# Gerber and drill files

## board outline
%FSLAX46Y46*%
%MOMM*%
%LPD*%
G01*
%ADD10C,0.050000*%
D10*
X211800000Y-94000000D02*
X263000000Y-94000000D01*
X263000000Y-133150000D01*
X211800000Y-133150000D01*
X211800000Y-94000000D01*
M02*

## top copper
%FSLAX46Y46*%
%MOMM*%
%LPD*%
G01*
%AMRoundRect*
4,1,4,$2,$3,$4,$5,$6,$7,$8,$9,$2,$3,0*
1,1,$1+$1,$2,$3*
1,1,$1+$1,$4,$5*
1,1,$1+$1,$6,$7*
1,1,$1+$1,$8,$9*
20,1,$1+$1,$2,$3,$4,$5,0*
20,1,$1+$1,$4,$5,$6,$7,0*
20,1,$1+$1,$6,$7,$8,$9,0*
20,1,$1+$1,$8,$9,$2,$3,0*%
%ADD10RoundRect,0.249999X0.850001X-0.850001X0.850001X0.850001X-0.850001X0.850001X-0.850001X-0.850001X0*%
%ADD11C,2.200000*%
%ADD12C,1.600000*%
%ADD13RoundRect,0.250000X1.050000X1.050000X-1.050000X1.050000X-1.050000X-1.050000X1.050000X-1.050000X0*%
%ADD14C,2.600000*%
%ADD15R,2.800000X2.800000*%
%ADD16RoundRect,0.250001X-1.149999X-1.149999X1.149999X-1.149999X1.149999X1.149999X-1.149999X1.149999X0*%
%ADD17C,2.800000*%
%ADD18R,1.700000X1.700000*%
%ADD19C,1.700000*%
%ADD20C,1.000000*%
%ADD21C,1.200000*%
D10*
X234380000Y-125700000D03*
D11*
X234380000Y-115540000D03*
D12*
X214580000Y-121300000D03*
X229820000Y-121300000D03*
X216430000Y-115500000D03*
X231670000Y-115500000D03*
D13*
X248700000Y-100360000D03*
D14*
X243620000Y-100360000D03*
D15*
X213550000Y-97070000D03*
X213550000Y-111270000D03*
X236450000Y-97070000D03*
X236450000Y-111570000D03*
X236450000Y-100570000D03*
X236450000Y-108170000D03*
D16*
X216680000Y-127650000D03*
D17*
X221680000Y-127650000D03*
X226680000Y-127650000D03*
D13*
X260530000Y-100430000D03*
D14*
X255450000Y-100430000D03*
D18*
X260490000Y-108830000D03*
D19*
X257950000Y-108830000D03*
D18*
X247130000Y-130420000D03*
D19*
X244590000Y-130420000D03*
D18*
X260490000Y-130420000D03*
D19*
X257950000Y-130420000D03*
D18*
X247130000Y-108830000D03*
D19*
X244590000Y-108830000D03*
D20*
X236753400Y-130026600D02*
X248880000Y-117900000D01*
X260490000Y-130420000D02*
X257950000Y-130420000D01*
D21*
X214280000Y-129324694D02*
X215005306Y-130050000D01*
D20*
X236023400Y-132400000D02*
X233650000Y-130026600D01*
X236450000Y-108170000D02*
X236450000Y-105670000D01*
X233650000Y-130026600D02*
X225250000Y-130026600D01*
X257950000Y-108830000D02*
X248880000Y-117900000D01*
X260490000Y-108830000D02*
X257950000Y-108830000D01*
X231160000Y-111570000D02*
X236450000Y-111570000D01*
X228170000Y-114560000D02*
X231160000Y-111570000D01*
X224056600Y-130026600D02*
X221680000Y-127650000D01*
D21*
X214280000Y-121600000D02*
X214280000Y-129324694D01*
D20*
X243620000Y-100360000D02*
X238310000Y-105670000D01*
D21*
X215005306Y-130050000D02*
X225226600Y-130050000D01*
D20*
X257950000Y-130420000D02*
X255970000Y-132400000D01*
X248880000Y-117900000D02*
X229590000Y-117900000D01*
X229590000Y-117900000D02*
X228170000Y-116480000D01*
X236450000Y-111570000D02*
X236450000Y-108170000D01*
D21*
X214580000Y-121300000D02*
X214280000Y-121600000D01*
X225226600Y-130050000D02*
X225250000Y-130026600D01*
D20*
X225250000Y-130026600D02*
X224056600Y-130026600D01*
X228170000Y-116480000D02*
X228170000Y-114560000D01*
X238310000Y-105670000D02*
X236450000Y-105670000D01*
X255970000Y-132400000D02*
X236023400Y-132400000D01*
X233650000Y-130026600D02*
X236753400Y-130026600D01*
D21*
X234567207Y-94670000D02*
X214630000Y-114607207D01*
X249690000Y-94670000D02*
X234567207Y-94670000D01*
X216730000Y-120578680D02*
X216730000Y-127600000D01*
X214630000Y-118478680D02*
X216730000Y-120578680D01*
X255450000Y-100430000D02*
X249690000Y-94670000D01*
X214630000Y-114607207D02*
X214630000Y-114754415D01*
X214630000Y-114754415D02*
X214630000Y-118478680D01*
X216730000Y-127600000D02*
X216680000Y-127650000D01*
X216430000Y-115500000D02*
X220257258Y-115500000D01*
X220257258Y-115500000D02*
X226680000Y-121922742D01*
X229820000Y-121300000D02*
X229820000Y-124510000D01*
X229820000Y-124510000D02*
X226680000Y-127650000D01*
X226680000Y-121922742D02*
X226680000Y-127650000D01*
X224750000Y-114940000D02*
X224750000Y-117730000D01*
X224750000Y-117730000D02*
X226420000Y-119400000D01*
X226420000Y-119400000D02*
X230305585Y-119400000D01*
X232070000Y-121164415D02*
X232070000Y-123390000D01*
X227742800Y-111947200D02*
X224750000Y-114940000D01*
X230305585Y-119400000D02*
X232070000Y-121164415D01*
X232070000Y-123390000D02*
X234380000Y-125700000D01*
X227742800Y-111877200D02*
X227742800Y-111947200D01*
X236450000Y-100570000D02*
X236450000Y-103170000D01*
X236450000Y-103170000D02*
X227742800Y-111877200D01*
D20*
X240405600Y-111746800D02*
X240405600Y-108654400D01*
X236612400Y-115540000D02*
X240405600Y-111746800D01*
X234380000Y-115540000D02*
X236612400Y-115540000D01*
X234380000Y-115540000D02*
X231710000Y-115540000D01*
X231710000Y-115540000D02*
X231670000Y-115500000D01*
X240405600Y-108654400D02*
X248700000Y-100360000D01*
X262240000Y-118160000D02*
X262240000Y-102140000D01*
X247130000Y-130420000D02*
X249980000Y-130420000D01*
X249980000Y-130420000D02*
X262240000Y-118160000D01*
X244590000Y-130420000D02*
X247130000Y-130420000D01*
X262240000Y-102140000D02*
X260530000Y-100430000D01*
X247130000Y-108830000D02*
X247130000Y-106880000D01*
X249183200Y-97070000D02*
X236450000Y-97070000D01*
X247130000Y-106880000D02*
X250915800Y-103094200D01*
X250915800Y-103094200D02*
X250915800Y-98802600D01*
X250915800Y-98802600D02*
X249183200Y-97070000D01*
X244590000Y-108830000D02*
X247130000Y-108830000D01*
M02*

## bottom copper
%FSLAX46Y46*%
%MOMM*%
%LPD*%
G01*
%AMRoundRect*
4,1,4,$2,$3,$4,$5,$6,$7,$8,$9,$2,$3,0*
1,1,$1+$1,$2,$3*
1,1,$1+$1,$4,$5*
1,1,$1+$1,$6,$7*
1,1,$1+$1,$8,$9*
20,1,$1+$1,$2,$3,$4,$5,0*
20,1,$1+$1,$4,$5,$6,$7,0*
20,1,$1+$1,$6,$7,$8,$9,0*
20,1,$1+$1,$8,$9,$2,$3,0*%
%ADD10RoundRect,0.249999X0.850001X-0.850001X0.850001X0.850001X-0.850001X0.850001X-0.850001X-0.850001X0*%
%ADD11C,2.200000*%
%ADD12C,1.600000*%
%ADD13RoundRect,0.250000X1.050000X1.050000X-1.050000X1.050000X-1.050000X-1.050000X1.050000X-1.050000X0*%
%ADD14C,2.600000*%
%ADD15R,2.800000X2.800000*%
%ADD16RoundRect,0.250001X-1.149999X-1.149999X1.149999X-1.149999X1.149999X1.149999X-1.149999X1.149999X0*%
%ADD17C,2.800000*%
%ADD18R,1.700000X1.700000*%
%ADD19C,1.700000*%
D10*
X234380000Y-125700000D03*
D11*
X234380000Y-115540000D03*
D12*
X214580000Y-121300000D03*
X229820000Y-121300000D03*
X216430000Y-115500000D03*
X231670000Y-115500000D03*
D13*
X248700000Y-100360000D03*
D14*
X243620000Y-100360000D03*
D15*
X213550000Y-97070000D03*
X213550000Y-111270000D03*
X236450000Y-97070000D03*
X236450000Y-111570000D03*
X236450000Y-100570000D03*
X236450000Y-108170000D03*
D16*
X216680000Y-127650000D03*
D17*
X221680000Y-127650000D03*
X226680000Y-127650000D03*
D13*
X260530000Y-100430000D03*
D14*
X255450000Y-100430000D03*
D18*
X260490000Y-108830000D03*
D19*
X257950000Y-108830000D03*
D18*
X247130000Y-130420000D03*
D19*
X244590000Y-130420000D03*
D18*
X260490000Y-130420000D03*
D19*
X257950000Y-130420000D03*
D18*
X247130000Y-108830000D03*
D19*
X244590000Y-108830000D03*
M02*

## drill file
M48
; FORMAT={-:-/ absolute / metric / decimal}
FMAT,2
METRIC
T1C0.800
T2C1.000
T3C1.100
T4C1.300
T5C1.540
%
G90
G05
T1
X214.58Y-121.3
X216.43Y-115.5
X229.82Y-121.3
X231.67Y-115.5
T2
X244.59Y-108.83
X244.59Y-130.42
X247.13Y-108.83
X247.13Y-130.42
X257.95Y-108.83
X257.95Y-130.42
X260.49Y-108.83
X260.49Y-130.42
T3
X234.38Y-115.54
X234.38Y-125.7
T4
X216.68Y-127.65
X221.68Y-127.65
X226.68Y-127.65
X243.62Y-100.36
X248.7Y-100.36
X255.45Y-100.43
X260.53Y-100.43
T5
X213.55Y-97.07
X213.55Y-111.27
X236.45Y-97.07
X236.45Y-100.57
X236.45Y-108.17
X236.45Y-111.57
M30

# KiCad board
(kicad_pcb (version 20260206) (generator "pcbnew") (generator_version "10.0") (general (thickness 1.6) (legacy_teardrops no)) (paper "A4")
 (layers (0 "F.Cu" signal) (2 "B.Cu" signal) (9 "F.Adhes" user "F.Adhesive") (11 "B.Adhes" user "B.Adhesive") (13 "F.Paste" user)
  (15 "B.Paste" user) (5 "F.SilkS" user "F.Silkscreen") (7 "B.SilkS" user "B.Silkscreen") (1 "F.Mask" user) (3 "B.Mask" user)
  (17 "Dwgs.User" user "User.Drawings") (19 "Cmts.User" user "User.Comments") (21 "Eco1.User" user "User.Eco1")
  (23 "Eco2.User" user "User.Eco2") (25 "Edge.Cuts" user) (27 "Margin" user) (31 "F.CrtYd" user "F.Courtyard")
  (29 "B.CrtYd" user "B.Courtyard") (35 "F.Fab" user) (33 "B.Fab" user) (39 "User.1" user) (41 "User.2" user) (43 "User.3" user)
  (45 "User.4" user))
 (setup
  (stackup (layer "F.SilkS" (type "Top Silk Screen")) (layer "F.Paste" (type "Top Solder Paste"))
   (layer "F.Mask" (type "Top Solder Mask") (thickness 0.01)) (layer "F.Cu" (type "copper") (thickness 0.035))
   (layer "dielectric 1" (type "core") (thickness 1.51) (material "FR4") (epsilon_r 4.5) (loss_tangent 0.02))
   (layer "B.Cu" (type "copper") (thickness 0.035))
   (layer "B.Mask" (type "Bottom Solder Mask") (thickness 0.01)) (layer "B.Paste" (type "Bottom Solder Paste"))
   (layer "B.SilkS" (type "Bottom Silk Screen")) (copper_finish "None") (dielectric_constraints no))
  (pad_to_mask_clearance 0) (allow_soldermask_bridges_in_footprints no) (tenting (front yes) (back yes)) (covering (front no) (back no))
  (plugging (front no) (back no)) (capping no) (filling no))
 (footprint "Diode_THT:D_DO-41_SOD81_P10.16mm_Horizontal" (layer "F.Cu") (at 234.38 125.7 90)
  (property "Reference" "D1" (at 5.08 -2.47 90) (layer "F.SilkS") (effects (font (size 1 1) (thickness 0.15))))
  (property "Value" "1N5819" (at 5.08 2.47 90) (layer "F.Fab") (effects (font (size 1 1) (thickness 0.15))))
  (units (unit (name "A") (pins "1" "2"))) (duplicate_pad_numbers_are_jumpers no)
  (pad "1" thru_hole roundrect (at 0 0 90) (size 2.2 2.2) (drill 1.1) (layers "*.Cu" "*.Mask") (remove_unused_layers no)
   (roundrect_rratio 0.113636) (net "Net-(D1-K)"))
  (pad "2" thru_hole circle (at 10.16 0 90) (size 2.2 2.2) (drill 1.1) (layers "*.Cu" "*.Mask") (remove_unused_layers no) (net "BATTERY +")))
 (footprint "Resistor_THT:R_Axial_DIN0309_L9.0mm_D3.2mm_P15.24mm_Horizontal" (layer "F.Cu") (at 214.58 121.3)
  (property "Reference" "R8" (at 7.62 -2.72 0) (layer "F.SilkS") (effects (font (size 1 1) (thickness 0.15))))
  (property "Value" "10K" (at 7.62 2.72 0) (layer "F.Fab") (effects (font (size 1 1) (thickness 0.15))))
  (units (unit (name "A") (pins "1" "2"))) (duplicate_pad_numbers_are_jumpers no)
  (pad "1" thru_hole circle (at 0 0) (size 1.6 1.6) (drill 0.8) (layers "*.Cu" "*.Mask") (remove_unused_layers no) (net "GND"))
  (pad "2" thru_hole circle (at 15.24 0) (size 1.6 1.6) (drill 0.8) (layers "*.Cu" "*.Mask") (remove_unused_layers no) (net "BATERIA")))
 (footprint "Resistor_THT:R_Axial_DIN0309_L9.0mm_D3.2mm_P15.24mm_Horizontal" (layer "F.Cu") (at 216.43 115.5)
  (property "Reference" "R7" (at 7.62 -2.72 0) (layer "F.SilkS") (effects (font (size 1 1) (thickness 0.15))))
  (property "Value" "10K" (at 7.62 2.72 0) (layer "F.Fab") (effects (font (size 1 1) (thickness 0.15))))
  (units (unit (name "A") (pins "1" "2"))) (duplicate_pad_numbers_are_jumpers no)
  (pad "1" thru_hole circle (at 0 0) (size 1.6 1.6) (drill 0.8) (layers "*.Cu" "*.Mask") (remove_unused_layers no) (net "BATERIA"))
  (pad "2" thru_hole circle (at 15.24 0) (size 1.6 1.6) (drill 0.8) (layers "*.Cu" "*.Mask") (remove_unused_layers no) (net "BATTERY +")))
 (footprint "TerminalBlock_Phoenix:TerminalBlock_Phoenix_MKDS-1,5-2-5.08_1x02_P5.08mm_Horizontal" (layer "F.Cu") (at 248.7 100.36 180)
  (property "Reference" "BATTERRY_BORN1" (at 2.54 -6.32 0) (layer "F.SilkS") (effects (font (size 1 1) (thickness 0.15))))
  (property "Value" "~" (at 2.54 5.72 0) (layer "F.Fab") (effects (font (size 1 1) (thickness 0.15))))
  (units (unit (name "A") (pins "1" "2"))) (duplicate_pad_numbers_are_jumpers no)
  (pad "1" thru_hole roundrect (at 0 0 180) (size 2.6 2.6) (drill 1.3) (layers "*.Cu" "*.Mask") (remove_unused_layers no)
   (roundrect_rratio 0.096154) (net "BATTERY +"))
  (pad "2" thru_hole circle (at 5.08 0 180) (size 2.6 2.6) (drill 1.3) (layers "*.Cu" "*.Mask") (remove_unused_layers no) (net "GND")))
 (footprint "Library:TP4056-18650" (layer "F.Cu") (at 211.85 95.37)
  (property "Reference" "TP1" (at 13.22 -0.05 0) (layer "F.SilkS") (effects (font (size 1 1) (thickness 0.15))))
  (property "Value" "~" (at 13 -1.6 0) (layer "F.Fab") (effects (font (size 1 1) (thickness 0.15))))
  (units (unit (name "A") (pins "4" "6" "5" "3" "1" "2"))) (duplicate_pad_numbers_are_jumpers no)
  (pad "1" thru_hole rect (at 1.7 1.7) (size 2.8 2.8) (drill 1.54) (layers "*.Cu" "*.Mask") (remove_unused_layers no)
   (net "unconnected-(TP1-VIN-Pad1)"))
  (pad "2" thru_hole rect (at 1.7 15.9) (size 2.8 2.8) (drill 1.54) (layers "*.Cu" "*.Mask") (remove_unused_layers no)
   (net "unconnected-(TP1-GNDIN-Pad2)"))
  (pad "3" thru_hole rect (at 24.6 1.7) (size 2.8 2.8) (drill 1.54) (layers "*.Cu" "*.Mask") (remove_unused_layers no) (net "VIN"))
  (pad "4" thru_hole rect (at 24.6 16.2) (size 2.8 2.8) (drill 1.54) (layers "*.Cu" "*.Mask") (remove_unused_layers no) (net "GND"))
  (pad "5" thru_hole rect (at 24.6 5.2) (size 2.8 2.8) (drill 1.54) (layers "*.Cu" "*.Mask") (remove_unused_layers no) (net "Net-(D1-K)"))
  (pad "6" thru_hole rect (at 24.6 12.8) (size 2.8 2.8) (drill 1.54) (layers "*.Cu" "*.Mask") (remove_unused_layers no) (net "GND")))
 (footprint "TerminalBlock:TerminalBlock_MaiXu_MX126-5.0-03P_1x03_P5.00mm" (layer "F.Cu") (at 216.68 127.65)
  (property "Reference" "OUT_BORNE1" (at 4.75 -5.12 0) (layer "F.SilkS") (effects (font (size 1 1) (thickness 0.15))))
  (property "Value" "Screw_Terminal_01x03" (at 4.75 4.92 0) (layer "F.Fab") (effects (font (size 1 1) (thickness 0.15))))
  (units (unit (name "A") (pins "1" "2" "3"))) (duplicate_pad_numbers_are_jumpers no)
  (pad "1" thru_hole roundrect (at 0 0) (size 2.8 2.8) (drill 1.3) (layers "*.Cu" "*.Mask") (remove_unused_layers no)
   (roundrect_rratio 0.089286) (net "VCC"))
  (pad "2" thru_hole circle (at 5 0) (size 2.8 2.8) (drill 1.3) (layers "*.Cu" "*.Mask") (remove_unused_layers no) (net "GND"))
  (pad "3" thru_hole circle (at 10 0) (size 2.8 2.8) (drill 1.3) (layers "*.Cu" "*.Mask") (remove_unused_layers no) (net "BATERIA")))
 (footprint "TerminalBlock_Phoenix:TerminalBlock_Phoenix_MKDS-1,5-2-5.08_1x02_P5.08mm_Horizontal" (layer "F.Cu") (at 260.53 100.43 180)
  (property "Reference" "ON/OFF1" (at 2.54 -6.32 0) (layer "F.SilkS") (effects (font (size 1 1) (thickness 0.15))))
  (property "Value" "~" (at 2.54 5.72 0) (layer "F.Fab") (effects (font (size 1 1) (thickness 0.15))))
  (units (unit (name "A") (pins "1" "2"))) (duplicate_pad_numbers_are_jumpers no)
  (pad "1" thru_hole roundrect (at 0 0 180) (size 2.6 2.6) (drill 1.3) (layers "*.Cu" "*.Mask") (remove_unused_layers no)
   (roundrect_rratio 0.096154) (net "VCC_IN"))
  (pad "2" thru_hole circle (at 5.08 0 180) (size 2.6 2.6) (drill 1.3) (layers "*.Cu" "*.Mask") (remove_unused_layers no) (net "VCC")))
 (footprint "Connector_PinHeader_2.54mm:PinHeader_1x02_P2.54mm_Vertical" (layer "B.Cu") (at 260.49 108.83 90)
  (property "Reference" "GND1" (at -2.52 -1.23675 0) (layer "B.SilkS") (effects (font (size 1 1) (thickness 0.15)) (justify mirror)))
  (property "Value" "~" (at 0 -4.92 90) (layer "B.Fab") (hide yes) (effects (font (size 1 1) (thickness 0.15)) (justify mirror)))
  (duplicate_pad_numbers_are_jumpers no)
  (pad "1" thru_hole rect (at 0 0 90) (size 1.7 1.7) (drill 1) (layers "*.Cu" "*.Mask") (remove_unused_layers no) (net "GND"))
  (pad "2" thru_hole circle (at 0 -2.54 90) (size 1.7 1.7) (drill 1) (layers "*.Cu" "*.Mask") (remove_unused_layers no) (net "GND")))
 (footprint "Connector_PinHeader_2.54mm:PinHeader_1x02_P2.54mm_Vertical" (layer "B.Cu") (at 247.13 130.42 90)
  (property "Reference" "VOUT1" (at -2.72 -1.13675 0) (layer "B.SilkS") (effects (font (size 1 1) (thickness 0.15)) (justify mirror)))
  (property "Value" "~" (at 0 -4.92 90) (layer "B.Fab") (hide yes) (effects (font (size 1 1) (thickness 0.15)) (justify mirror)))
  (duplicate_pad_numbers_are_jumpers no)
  (pad "1" thru_hole rect (at 0 0 90) (size 1.7 1.7) (drill 1) (layers "*.Cu" "*.Mask") (remove_unused_layers no) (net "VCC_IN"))
  (pad "2" thru_hole circle (at 0 -2.54 90) (size 1.7 1.7) (drill 1) (layers "*.Cu" "*.Mask") (remove_unused_layers no) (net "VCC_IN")))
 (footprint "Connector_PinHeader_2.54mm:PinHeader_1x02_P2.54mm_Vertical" (layer "B.Cu") (at 260.49 130.42 90)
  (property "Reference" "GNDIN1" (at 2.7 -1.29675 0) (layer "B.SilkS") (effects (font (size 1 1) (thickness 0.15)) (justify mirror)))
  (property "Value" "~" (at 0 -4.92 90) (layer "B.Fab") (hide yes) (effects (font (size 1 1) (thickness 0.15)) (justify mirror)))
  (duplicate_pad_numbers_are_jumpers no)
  (pad "1" thru_hole rect (at 0 0 90) (size 1.7 1.7) (drill 1) (layers "*.Cu" "*.Mask") (remove_unused_layers no) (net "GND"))
  (pad "2" thru_hole circle (at 0 -2.54 90) (size 1.7 1.7) (drill 1) (layers "*.Cu" "*.Mask") (remove_unused_layers no) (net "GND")))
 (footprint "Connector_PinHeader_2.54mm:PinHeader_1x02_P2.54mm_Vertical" (layer "B.Cu") (at 247.13 108.83 90)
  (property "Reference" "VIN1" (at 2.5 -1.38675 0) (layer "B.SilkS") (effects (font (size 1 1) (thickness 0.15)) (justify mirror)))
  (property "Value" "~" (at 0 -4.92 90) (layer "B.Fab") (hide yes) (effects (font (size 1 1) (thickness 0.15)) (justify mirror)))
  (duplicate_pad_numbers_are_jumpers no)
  (pad "1" thru_hole rect (at 0 0 90) (size 1.7 1.7) (drill 1) (layers "*.Cu" "*.Mask") (remove_unused_layers no) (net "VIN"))
  (pad "2" thru_hole circle (at 0 -2.54 90) (size 1.7 1.7) (drill 1) (layers "*.Cu" "*.Mask") (remove_unused_layers no) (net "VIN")))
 (gr_rect (start 211.8 94) (end 263 133.15) (stroke (width 0.05) (type default)) (fill no) (layer "Edge.Cuts"))
 (segment (start 236.7534 130.0266) (end 248.88 117.9) (width 1) (layer "F.Cu") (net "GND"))
 (segment (start 260.49 130.42) (end 257.95 130.42) (width 1) (layer "F.Cu") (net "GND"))
 (segment (start 214.28 129.324694) (end 215.005306 130.05) (width 1.2) (layer "F.Cu") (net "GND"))
 (segment (start 236.0234 132.4) (end 233.65 130.0266) (width 1) (layer "F.Cu") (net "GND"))
 (segment (start 236.45 108.17) (end 236.45 105.67) (width 1) (layer "F.Cu") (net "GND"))
 (segment (start 233.65 130.0266) (end 225.25 130.0266) (width 1) (layer "F.Cu") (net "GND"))
 (segment (start 257.95 108.83) (end 248.88 117.9) (width 1) (layer "F.Cu") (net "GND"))
 (segment (start 260.49 108.83) (end 257.95 108.83) (width 1) (layer "F.Cu") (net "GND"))
 (segment (start 231.16 111.57) (end 236.45 111.57) (width 1) (layer "F.Cu") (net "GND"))
 (segment (start 228.17 114.56) (end 231.16 111.57) (width 1) (layer "F.Cu") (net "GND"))
 (segment (start 224.0566 130.0266) (end 221.68 127.65) (width 1) (layer "F.Cu") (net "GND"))
 (segment (start 214.28 121.6) (end 214.28 129.324694) (width 1.2) (layer "F.Cu") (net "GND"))
 (segment (start 243.62 100.36) (end 238.31 105.67) (width 1) (layer "F.Cu") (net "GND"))
 (segment (start 215.005306 130.05) (end 225.2266 130.05) (width 1.2) (layer "F.Cu") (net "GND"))
 (segment (start 257.95 130.42) (end 255.97 132.4) (width 1) (layer "F.Cu") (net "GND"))
 (segment (start 248.88 117.9) (end 229.59 117.9) (width 1) (layer "F.Cu") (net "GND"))
 (segment (start 229.59 117.9) (end 228.17 116.48) (width 1) (layer "F.Cu") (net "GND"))
 (segment (start 236.45 111.57) (end 236.45 108.17) (width 1) (layer "F.Cu") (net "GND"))
 (segment (start 214.58 121.3) (end 214.28 121.6) (width 1.2) (layer "F.Cu") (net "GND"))
 (segment (start 225.2266 130.05) (end 225.25 130.0266) (width 1.2) (layer "F.Cu") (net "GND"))
 (segment (start 225.25 130.0266) (end 224.0566 130.0266) (width 1) (layer "F.Cu") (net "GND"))
 (segment (start 228.17 116.48) (end 228.17 114.56) (width 1) (layer "F.Cu") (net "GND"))
 (segment (start 238.31 105.67) (end 236.45 105.67) (width 1) (layer "F.Cu") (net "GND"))
 (segment (start 255.97 132.4) (end 236.0234 132.4) (width 1) (layer "F.Cu") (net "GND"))
 (segment (start 233.65 130.0266) (end 236.7534 130.0266) (width 1) (layer "F.Cu") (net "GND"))
 (segment (start 234.567207 94.67) (end 214.63 114.607207) (width 1.2) (layer "F.Cu") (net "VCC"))
 (segment (start 249.69 94.67) (end 234.567207 94.67) (width 1.2) (layer "F.Cu") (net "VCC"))
 (segment (start 216.73 120.57868) (end 216.73 127.6) (width 1.2) (layer "F.Cu") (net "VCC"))
 (segment (start 214.63 118.47868) (end 216.73 120.57868) (width 1.2) (layer "F.Cu") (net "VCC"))
 (segment (start 255.45 100.43) (end 249.69 94.67) (width 1.2) (layer "F.Cu") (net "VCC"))
 (segment (start 214.63 114.607207) (end 214.63 114.754415) (width 1.2) (layer "F.Cu") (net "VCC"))
 (segment (start 214.63 114.754415) (end 214.63 118.47868) (width 1.2) (layer "F.Cu") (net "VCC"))
 (segment (start 216.73 127.6) (end 216.68 127.65) (width 1.2) (layer "F.Cu") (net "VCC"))
 (segment (start 216.43 115.5) (end 220.257258 115.5) (width 1.2) (layer "F.Cu") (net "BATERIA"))
 (segment (start 220.257258 115.5) (end 226.68 121.922742) (width 1.2) (layer "F.Cu") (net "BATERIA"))
 (segment (start 229.82 121.3) (end 229.82 124.51) (width 1.2) (layer "F.Cu") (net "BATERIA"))
 (segment (start 229.82 124.51) (end 226.68 127.65) (width 1.2) (layer "F.Cu") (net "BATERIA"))
 (segment (start 226.68 121.922742) (end 226.68 127.65) (width 1.2) (layer "F.Cu") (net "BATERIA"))
 (segment (start 224.75 114.94) (end 224.75 117.73) (width 1.2) (layer "F.Cu") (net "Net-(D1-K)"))
 (segment (start 224.75 117.73) (end 226.42 119.4) (width 1.2) (layer "F.Cu") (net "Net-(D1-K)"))
 (segment (start 226.42 119.4) (end 230.305585 119.4) (width 1.2) (layer "F.Cu") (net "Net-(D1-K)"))
 (segment (start 232.07 121.164415) (end 232.07 123.39) (width 1.2) (layer "F.Cu") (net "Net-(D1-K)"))
 (segment (start 227.7428 111.9472) (end 224.75 114.94) (width 1.2) (layer "F.Cu") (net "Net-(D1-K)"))
 (segment (start 230.305585 119.4) (end 232.07 121.164415) (width 1.2) (layer "F.Cu") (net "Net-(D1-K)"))
 (segment (start 232.07 123.39) (end 234.38 125.7) (width 1.2) (layer "F.Cu") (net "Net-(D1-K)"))
 (segment (start 227.7428 111.8772) (end 227.7428 111.9472) (width 1.2) (layer "F.Cu") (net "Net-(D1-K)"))
 (segment (start 236.45 100.57) (end 236.45 103.17) (width 1.2) (layer "F.Cu") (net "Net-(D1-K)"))
 (segment (start 236.45 103.17) (end 227.7428 111.8772) (width 1.2) (layer "F.Cu") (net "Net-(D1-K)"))
 (segment (start 240.4056 111.7468) (end 240.4056 108.6544) (width 1) (layer "F.Cu") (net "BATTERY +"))
 (segment (start 236.6124 115.54) (end 240.4056 111.7468) (width 1) (layer "F.Cu") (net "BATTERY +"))
 (segment (start 234.38 115.54) (end 236.6124 115.54) (width 1) (layer "F.Cu") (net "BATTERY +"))
 (segment (start 234.38 115.54) (end 231.71 115.54) (width 1) (layer "F.Cu") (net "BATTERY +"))
 (segment (start 231.71 115.54) (end 231.67 115.5) (width 1) (layer "F.Cu") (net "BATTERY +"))
 (segment (start 240.4056 108.6544) (end 248.7 100.36) (width 1) (layer "F.Cu") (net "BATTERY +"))
 (segment (start 262.24 118.16) (end 262.24 102.14) (width 1) (layer "F.Cu") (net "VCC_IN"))
 (segment (start 247.13 130.42) (end 249.98 130.42) (width 1) (layer "F.Cu") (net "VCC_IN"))
 (segment (start 249.98 130.42) (end 262.24 118.16) (width 1) (layer "F.Cu") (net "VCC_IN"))
 (segment (start 244.59 130.42) (end 247.13 130.42) (width 1) (layer "F.Cu") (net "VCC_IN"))
 (segment (start 262.24 102.14) (end 260.53 100.43) (width 1) (layer "F.Cu") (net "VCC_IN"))
 (segment (start 247.13 108.83) (end 247.13 106.88) (width 1) (layer "F.Cu") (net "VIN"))
 (segment (start 249.1832 97.07) (end 236.45 97.07) (width 1) (layer "F.Cu") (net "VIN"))
 (segment (start 247.13 106.88) (end 250.9158 103.0942) (width 1) (layer "F.Cu") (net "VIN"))
 (segment (start 250.9158 103.0942) (end 250.9158 98.8026) (width 1) (layer "F.Cu") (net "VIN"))
 (segment (start 250.9158 98.8026) (end 249.1832 97.07) (width 1) (layer "F.Cu") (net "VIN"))
 (segment (start 244.59 108.83) (end 247.13 108.83) (width 1) (layer "F.Cu") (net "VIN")))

